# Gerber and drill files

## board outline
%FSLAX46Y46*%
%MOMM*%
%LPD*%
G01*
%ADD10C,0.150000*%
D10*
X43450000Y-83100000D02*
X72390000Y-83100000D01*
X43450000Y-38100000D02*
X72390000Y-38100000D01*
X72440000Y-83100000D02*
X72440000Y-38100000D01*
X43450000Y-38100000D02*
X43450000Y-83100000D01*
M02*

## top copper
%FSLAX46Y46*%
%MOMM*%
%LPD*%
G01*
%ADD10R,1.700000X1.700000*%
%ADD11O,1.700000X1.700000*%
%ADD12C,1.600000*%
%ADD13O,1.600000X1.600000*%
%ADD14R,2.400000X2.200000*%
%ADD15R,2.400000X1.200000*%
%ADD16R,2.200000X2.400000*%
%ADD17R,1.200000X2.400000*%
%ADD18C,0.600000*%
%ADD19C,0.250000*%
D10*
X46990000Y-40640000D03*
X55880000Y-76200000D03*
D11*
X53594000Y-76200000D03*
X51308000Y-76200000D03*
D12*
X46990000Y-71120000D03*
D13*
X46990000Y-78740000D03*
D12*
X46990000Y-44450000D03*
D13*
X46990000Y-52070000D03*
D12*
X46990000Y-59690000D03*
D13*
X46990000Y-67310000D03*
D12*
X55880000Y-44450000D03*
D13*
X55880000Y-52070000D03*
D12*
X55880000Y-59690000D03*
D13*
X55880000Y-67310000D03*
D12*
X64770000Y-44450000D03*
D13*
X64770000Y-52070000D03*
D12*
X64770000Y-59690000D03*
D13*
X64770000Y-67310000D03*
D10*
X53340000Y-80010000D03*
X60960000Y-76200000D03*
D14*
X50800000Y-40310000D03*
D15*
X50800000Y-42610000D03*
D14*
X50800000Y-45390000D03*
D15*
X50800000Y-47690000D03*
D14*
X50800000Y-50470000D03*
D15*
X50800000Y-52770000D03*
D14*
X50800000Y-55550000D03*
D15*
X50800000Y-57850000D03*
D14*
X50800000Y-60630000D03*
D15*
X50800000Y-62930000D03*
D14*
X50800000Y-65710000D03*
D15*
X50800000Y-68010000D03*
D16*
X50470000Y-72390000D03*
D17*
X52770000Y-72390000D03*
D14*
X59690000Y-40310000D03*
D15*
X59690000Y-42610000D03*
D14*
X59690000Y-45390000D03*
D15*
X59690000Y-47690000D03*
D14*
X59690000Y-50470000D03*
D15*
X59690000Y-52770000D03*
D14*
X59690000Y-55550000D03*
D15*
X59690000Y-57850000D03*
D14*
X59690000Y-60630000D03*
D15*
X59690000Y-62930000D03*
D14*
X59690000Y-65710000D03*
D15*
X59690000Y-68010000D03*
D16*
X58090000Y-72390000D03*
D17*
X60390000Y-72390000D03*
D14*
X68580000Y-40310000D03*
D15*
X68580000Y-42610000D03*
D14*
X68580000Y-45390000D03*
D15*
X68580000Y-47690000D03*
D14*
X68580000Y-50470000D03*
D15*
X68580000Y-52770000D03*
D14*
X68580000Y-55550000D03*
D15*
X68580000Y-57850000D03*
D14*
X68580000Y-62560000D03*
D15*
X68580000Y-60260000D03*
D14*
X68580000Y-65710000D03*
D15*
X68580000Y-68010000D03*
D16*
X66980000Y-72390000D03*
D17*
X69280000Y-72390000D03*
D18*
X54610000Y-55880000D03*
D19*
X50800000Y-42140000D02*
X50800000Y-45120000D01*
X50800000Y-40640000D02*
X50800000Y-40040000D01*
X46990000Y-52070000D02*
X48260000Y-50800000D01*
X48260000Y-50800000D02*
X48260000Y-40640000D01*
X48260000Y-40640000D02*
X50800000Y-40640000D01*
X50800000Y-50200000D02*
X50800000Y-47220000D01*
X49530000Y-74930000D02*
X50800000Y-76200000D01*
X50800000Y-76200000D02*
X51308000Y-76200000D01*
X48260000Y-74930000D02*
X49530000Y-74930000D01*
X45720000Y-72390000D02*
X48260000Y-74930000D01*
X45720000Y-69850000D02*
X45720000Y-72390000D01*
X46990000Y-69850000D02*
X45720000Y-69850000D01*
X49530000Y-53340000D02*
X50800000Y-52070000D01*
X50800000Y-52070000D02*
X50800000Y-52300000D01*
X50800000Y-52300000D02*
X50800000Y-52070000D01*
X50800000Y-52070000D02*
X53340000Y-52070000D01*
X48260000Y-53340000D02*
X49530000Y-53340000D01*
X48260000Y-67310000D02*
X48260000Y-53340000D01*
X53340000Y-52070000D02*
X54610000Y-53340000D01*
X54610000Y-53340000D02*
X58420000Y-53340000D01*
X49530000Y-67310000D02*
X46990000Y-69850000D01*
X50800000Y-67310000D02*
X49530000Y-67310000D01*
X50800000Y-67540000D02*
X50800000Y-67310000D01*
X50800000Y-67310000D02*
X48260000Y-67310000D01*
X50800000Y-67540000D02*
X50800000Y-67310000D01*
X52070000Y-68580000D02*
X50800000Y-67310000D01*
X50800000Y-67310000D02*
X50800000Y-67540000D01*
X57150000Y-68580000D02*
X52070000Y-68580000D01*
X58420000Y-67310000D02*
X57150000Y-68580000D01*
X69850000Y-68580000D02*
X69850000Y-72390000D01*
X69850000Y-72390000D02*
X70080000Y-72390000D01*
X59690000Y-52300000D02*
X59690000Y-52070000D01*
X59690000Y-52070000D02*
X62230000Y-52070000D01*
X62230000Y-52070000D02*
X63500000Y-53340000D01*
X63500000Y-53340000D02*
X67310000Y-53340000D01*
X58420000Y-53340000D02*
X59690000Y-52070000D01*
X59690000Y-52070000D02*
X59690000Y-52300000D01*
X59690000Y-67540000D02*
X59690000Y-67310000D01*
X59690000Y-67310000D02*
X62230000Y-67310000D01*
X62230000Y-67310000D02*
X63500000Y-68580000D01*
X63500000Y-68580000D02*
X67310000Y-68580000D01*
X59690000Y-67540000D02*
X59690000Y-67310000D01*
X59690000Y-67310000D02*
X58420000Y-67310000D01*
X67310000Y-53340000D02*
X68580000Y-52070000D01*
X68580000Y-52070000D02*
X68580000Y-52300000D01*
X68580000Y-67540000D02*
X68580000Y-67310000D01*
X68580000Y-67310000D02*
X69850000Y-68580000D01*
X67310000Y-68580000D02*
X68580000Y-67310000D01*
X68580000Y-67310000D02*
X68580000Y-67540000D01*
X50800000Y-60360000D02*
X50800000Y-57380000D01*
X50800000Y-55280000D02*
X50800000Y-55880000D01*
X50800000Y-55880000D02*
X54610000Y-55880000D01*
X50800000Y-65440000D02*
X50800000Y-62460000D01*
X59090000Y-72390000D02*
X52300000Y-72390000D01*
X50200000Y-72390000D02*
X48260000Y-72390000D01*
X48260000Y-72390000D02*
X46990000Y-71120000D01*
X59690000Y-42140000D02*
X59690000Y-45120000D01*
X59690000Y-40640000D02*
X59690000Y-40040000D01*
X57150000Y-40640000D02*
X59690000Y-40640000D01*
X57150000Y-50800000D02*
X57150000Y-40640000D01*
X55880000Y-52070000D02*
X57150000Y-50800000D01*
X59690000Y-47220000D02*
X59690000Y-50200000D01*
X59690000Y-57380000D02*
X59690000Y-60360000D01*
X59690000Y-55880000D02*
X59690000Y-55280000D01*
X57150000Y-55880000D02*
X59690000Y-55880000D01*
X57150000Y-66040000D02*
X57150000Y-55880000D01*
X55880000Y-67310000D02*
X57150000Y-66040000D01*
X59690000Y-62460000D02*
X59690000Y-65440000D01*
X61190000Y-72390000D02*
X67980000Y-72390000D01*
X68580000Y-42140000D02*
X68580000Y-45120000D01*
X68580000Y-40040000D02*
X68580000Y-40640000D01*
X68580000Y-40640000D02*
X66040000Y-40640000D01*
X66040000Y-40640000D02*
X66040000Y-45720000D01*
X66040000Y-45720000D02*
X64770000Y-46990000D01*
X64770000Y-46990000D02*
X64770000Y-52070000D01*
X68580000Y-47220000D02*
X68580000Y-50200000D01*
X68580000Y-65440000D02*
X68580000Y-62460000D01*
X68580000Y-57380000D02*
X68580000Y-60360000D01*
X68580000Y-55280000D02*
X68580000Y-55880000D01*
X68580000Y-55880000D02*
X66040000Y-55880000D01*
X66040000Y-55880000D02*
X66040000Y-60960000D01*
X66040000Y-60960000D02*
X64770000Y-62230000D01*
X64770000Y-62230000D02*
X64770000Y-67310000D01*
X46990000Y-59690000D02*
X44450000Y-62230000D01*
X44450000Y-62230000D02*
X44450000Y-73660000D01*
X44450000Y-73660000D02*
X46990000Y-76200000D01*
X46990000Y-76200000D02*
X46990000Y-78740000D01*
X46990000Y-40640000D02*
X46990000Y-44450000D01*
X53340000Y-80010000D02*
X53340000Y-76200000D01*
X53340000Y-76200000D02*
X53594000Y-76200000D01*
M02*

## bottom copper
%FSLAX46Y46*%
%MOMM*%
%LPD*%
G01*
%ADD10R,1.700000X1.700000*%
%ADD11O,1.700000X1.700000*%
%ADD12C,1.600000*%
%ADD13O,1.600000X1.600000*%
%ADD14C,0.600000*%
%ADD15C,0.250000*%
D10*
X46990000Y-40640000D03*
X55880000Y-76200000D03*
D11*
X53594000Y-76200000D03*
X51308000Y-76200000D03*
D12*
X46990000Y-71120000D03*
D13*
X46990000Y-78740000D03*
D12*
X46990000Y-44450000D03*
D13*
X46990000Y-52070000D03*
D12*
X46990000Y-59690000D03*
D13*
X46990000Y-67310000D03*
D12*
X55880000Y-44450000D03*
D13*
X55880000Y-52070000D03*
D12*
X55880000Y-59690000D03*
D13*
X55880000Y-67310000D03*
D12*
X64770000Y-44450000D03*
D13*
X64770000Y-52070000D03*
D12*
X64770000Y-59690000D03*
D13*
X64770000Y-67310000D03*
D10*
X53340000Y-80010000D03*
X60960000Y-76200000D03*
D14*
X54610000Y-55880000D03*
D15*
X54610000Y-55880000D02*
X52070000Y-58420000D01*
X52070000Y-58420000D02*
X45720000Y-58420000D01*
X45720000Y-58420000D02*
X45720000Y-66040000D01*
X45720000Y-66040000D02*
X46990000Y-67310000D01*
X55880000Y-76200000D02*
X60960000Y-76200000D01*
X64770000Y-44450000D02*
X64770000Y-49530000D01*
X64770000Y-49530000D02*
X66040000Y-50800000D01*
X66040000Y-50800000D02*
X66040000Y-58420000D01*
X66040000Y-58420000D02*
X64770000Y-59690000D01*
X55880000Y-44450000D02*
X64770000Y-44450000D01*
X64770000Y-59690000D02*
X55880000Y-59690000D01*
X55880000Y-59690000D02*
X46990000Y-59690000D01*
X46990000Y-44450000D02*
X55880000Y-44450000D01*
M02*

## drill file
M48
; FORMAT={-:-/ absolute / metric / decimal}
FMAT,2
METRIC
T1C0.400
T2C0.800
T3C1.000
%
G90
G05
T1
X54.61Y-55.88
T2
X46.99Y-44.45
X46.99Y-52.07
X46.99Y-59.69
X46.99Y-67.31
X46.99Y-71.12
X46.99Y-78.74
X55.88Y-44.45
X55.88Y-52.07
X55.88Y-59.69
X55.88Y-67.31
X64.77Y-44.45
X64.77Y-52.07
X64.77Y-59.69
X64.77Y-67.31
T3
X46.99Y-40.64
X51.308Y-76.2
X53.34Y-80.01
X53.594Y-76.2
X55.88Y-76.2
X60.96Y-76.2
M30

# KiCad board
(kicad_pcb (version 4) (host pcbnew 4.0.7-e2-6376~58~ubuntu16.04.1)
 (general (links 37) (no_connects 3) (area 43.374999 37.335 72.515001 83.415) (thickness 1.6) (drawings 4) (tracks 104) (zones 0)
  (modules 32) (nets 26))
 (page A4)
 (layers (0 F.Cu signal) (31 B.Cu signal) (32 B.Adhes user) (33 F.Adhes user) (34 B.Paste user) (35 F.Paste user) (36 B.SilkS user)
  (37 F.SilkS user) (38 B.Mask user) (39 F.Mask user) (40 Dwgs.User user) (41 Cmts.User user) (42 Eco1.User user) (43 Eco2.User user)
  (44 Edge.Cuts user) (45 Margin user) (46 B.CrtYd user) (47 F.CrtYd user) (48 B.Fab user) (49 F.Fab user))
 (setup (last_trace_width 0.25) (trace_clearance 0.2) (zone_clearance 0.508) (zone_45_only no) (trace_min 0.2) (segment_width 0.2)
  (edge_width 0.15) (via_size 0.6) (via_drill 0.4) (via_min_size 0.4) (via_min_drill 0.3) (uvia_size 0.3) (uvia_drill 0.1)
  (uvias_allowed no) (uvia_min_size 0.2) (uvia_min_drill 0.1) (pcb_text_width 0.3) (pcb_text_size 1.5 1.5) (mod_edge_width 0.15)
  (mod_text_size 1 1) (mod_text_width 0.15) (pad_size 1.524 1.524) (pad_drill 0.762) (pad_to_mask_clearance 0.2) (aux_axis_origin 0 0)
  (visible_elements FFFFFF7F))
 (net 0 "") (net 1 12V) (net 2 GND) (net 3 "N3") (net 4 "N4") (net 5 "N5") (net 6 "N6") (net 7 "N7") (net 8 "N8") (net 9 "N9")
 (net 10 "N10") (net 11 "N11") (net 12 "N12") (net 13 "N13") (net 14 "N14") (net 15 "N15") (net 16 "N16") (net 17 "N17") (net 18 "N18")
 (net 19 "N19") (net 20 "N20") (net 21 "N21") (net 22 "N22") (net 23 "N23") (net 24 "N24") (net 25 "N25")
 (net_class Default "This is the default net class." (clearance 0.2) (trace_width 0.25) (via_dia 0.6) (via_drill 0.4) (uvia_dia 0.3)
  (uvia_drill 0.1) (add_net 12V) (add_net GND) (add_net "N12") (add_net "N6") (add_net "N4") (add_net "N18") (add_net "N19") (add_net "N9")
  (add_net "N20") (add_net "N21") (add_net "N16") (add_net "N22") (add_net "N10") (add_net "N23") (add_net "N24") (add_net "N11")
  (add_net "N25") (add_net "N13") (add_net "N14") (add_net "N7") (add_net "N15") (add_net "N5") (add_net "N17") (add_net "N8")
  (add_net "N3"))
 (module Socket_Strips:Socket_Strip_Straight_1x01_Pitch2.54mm (layer F.Cu) (at 46.99 40.64)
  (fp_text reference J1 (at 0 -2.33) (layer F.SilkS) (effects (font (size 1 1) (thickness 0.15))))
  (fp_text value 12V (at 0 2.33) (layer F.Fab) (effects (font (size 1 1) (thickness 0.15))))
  (pad 1 thru_hole rect (at 0 0) (size 1.7 1.7) (drill 1) (layers *.Cu *.Mask) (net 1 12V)))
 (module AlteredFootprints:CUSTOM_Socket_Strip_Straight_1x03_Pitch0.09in (layer F.Cu) (at 55.88 76.2 270)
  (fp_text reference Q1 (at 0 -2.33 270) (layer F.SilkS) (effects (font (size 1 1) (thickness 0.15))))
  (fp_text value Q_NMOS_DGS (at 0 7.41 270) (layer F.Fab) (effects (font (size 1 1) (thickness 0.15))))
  (pad 1 thru_hole rect (at 0 0 270) (size 1.7 1.7) (drill 1) (layers *.Cu *.Mask) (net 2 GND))
  (pad 2 thru_hole oval (at 0 2.286 270) (size 1.7 1.7) (drill 1) (layers *.Cu *.Mask) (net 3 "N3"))
  (pad 3 thru_hole oval (at 0 4.572 270) (size 1.7 1.7) (drill 1) (layers *.Cu *.Mask) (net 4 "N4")))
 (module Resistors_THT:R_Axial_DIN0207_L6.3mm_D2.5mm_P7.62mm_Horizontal (layer F.Cu) (at 46.99 71.12 270)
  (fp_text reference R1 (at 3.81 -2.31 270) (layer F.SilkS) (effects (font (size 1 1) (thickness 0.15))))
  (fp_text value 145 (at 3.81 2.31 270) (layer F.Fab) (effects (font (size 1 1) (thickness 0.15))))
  (pad 1 thru_hole circle (at 0 0 270) (size 1.6 1.6) (drill 0.8) (layers *.Cu *.Mask) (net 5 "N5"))
  (pad 2 thru_hole oval (at 7.62 0 270) (size 1.6 1.6) (drill 0.8) (layers *.Cu *.Mask) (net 1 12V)))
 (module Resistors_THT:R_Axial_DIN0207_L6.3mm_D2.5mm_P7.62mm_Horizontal (layer F.Cu) (at 46.99 44.45 270)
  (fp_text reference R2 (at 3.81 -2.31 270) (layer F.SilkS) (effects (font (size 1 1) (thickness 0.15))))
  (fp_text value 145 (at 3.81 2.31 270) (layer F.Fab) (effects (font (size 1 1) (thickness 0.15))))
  (pad 1 thru_hole circle (at 0 0 270) (size 1.6 1.6) (drill 0.8) (layers *.Cu *.Mask) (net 1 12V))
  (pad 2 thru_hole oval (at 7.62 0 270) (size 1.6 1.6) (drill 0.8) (layers *.Cu *.Mask) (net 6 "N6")))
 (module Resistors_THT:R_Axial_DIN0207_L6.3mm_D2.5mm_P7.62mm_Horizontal (layer F.Cu) (at 46.99 59.69 270)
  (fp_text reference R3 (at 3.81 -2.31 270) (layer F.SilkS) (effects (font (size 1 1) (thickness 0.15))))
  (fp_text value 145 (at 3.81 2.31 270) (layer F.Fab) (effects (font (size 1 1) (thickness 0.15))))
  (pad 1 thru_hole circle (at 0 0 270) (size 1.6 1.6) (drill 0.8) (layers *.Cu *.Mask) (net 1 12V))
  (pad 2 thru_hole oval (at 7.62 0 270) (size 1.6 1.6) (drill 0.8) (layers *.Cu *.Mask) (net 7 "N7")))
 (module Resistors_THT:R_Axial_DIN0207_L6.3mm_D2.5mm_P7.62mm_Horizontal (layer F.Cu) (at 55.88 44.45 270)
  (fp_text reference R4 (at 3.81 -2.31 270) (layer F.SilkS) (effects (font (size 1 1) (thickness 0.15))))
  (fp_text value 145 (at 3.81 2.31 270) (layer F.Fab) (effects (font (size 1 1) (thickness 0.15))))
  (pad 1 thru_hole circle (at 0 0 270) (size 1.6 1.6) (drill 0.8) (layers *.Cu *.Mask) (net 1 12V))
  (pad 2 thru_hole oval (at 7.62 0 270) (size 1.6 1.6) (drill 0.8) (layers *.Cu *.Mask) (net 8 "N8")))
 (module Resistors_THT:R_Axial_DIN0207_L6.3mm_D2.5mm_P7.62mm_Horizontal (layer F.Cu) (at 55.88 59.69 270)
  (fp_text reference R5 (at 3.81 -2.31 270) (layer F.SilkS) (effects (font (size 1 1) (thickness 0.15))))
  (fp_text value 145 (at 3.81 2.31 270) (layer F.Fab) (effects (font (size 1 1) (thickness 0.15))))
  (pad 1 thru_hole circle (at 0 0 270) (size 1.6 1.6) (drill 0.8) (layers *.Cu *.Mask) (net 1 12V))
  (pad 2 thru_hole oval (at 7.62 0 270) (size 1.6 1.6) (drill 0.8) (layers *.Cu *.Mask) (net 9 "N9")))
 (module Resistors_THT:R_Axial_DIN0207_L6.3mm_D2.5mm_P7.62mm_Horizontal (layer F.Cu) (at 64.77 44.45 270)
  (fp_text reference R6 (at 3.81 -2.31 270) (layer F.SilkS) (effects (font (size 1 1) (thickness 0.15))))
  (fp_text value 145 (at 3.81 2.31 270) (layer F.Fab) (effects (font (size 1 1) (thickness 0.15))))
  (pad 1 thru_hole circle (at 0 0 270) (size 1.6 1.6) (drill 0.8) (layers *.Cu *.Mask) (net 1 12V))
  (pad 2 thru_hole oval (at 7.62 0 270) (size 1.6 1.6) (drill 0.8) (layers *.Cu *.Mask) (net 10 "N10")))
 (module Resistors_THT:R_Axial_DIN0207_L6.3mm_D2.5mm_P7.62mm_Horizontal (layer F.Cu) (at 64.77 59.69 270)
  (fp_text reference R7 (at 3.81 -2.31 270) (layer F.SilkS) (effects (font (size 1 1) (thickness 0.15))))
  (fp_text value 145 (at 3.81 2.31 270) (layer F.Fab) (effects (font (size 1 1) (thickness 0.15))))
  (pad 1 thru_hole circle (at 0 0 270) (size 1.6 1.6) (drill 0.8) (layers *.Cu *.Mask) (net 1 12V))
  (pad 2 thru_hole oval (at 7.62 0 270) (size 1.6 1.6) (drill 0.8) (layers *.Cu *.Mask) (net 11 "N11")))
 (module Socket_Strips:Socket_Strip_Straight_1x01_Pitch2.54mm (layer F.Cu) (at 53.34 80.01)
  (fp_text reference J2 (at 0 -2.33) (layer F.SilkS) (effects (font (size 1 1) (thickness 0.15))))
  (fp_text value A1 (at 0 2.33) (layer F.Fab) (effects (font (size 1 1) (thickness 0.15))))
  (pad 1 thru_hole rect (at 0 0) (size 1.7 1.7) (drill 1) (layers *.Cu *.Mask) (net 3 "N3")))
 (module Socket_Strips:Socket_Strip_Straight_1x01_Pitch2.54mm (layer F.Cu) (at 60.96 76.2)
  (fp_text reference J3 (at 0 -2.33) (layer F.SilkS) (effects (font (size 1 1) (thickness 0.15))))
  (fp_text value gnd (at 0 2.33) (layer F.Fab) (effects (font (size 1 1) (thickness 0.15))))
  (pad 1 thru_hole rect (at 0 0) (size 1.7 1.7) (drill 1) (layers *.Cu *.Mask) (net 2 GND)))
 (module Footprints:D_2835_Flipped (layer F.Cu) (at 50.8 41.91 90)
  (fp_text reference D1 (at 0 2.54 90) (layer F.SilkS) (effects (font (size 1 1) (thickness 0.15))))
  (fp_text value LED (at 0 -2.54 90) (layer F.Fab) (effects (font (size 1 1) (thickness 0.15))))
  (pad 2 smd rect (at 1.6 0 90) (size 2.2 2.4) (layers F.Cu F.Paste F.Mask) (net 6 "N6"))
  (pad 1 smd rect (at -0.7 0 90) (size 1.2 2.4) (layers F.Cu F.Paste F.Mask) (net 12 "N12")))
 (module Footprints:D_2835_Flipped (layer F.Cu) (at 50.8 46.99 90)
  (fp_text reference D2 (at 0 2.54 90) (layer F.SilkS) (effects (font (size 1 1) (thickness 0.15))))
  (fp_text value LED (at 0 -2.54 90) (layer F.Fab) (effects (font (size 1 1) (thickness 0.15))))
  (pad 2 smd rect (at 1.6 0 90) (size 2.2 2.4) (layers F.Cu F.Paste F.Mask) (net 12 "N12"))
  (pad 1 smd rect (at -0.7 0 90) (size 1.2 2.4) (layers F.Cu F.Paste F.Mask) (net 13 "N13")))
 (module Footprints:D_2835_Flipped (layer F.Cu) (at 50.8 52.07 90)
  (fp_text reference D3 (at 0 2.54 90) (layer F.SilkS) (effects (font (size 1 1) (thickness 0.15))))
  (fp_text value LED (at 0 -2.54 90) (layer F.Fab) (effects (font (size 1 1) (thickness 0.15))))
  (pad 2 smd rect (at 1.6 0 90) (size 2.2 2.4) (layers F.Cu F.Paste F.Mask) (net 13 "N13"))
  (pad 1 smd rect (at -0.7 0 90) (size 1.2 2.4) (layers F.Cu F.Paste F.Mask) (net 4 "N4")))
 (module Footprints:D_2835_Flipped (layer F.Cu) (at 50.8 57.15 90)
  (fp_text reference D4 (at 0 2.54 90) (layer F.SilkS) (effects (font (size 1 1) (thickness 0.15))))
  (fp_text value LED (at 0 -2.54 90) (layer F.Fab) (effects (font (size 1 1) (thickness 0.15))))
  (pad 2 smd rect (at 1.6 0 90) (size 2.2 2.4) (layers F.Cu F.Paste F.Mask) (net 7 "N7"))
  (pad 1 smd rect (at -0.7 0 90) (size 1.2 2.4) (layers F.Cu F.Paste F.Mask) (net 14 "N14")))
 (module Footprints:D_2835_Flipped (layer F.Cu) (at 50.8 62.23 90)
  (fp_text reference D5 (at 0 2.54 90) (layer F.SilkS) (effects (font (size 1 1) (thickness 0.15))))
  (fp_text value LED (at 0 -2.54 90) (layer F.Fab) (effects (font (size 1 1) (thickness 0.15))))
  (pad 2 smd rect (at 1.6 0 90) (size 2.2 2.4) (layers F.Cu F.Paste F.Mask) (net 14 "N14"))
  (pad 1 smd rect (at -0.7 0 90) (size 1.2 2.4) (layers F.Cu F.Paste F.Mask) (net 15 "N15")))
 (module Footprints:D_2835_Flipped (layer F.Cu) (at 50.8 67.31 90)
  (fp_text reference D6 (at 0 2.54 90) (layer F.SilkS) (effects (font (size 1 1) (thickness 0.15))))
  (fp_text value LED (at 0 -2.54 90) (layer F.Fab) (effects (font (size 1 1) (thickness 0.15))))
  (pad 2 smd rect (at 1.6 0 90) (size 2.2 2.4) (layers F.Cu F.Paste F.Mask) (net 15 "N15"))
  (pad 1 smd rect (at -0.7 0 90) (size 1.2 2.4) (layers F.Cu F.Paste F.Mask) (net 4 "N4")))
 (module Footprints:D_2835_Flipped (layer F.Cu) (at 52.07 72.39 180)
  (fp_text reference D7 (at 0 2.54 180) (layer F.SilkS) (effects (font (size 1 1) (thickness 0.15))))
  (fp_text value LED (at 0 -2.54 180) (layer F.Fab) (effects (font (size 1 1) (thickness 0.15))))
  (pad 2 smd rect (at 1.6 0 180) (size 2.2 2.4) (layers F.Cu F.Paste F.Mask) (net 5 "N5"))
  (pad 1 smd rect (at -0.7 0 180) (size 1.2 2.4) (layers F.Cu F.Paste F.Mask) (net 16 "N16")))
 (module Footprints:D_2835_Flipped (layer F.Cu) (at 59.69 41.91 90)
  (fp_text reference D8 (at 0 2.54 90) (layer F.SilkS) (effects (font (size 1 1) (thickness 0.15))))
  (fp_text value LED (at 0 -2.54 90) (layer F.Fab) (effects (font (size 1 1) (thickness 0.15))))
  (pad 2 smd rect (at 1.6 0 90) (size 2.2 2.4) (layers F.Cu F.Paste F.Mask) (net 8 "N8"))
  (pad 1 smd rect (at -0.7 0 90) (size 1.2 2.4) (layers F.Cu F.Paste F.Mask) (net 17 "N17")))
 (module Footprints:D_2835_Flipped (layer F.Cu) (at 59.69 46.99 90)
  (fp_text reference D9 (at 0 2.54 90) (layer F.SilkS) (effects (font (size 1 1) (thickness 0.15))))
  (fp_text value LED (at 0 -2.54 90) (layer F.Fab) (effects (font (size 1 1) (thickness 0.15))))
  (pad 2 smd rect (at 1.6 0 90) (size 2.2 2.4) (layers F.Cu F.Paste F.Mask) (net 17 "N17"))
  (pad 1 smd rect (at -0.7 0 90) (size 1.2 2.4) (layers F.Cu F.Paste F.Mask) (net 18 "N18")))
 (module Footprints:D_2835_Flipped (layer F.Cu) (at 59.69 52.07 90)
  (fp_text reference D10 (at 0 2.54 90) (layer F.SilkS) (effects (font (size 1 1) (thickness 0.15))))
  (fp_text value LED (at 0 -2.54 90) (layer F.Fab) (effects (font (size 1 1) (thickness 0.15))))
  (pad 2 smd rect (at 1.6 0 90) (size 2.2 2.4) (layers F.Cu F.Paste F.Mask) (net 18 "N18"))
  (pad 1 smd rect (at -0.7 0 90) (size 1.2 2.4) (layers F.Cu F.Paste F.Mask) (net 4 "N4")))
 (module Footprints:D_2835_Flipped (layer F.Cu) (at 59.69 57.15 90)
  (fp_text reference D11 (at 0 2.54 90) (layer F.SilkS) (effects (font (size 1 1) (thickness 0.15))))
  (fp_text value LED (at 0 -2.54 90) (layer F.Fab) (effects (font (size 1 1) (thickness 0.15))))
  (pad 2 smd rect (at 1.6 0 90) (size 2.2 2.4) (layers F.Cu F.Paste F.Mask) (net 9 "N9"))
  (pad 1 smd rect (at -0.7 0 90) (size 1.2 2.4) (layers F.Cu F.Paste F.Mask) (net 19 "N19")))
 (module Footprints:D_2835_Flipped (layer F.Cu) (at 59.69 62.23 90)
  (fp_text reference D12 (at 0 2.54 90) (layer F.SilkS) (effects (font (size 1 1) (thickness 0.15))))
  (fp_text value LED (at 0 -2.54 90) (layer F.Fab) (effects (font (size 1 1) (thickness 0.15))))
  (pad 2 smd rect (at 1.6 0 90) (size 2.2 2.4) (layers F.Cu F.Paste F.Mask) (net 19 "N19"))
  (pad 1 smd rect (at -0.7 0 90) (size 1.2 2.4) (layers F.Cu F.Paste F.Mask) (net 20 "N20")))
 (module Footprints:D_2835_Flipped (layer F.Cu) (at 59.69 67.31 90)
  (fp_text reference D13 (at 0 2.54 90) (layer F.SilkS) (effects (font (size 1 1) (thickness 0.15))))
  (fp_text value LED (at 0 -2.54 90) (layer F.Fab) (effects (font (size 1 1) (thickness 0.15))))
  (pad 2 smd rect (at 1.6 0 90) (size 2.2 2.4) (layers F.Cu F.Paste F.Mask) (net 20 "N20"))
  (pad 1 smd rect (at -0.7 0 90) (size 1.2 2.4) (layers F.Cu F.Paste F.Mask) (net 4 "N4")))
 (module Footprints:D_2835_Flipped (layer F.Cu) (at 59.69 72.39 180)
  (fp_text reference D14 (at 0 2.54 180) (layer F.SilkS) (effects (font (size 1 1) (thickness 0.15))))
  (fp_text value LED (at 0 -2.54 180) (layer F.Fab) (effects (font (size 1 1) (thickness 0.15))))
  (pad 2 smd rect (at 1.6 0 180) (size 2.2 2.4) (layers F.Cu F.Paste F.Mask) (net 16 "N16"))
  (pad 1 smd rect (at -0.7 0 180) (size 1.2 2.4) (layers F.Cu F.Paste F.Mask) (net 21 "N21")))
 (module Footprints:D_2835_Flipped (layer F.Cu) (at 68.58 41.91 90)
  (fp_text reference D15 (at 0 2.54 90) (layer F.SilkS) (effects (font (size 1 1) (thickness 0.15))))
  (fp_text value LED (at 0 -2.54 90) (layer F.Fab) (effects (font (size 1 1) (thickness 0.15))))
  (pad 2 smd rect (at 1.6 0 90) (size 2.2 2.4) (layers F.Cu F.Paste F.Mask) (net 10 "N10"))
  (pad 1 smd rect (at -0.7 0 90) (size 1.2 2.4) (layers F.Cu F.Paste F.Mask) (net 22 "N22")))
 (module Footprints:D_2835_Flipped (layer F.Cu) (at 68.58 46.99 90)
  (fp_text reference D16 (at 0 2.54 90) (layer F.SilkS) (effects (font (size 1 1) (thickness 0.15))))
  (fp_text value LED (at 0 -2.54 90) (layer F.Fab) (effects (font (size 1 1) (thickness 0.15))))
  (pad 2 smd rect (at 1.6 0 90) (size 2.2 2.4) (layers F.Cu F.Paste F.Mask) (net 22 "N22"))
  (pad 1 smd rect (at -0.7 0 90) (size 1.2 2.4) (layers F.Cu F.Paste F.Mask) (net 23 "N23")))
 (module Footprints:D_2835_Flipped (layer F.Cu) (at 68.58 52.07 90)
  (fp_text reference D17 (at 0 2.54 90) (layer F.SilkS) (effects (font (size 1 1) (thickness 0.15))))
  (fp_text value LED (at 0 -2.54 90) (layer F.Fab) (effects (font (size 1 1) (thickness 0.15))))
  (pad 2 smd rect (at 1.6 0 90) (size 2.2 2.4) (layers F.Cu F.Paste F.Mask) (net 23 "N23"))
  (pad 1 smd rect (at -0.7 0 90) (size 1.2 2.4) (layers F.Cu F.Paste F.Mask) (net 4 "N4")))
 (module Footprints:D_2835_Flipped (layer F.Cu) (at 68.58 57.15 90)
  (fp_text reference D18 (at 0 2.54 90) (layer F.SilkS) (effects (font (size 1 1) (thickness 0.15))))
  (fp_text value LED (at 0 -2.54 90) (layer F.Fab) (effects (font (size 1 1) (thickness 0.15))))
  (pad 2 smd rect (at 1.6 0 90) (size 2.2 2.4) (layers F.Cu F.Paste F.Mask) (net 11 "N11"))
  (pad 1 smd rect (at -0.7 0 90) (size 1.2 2.4) (layers F.Cu F.Paste F.Mask) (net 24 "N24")))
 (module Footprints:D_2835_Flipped (layer F.Cu) (at 68.58 60.96 270)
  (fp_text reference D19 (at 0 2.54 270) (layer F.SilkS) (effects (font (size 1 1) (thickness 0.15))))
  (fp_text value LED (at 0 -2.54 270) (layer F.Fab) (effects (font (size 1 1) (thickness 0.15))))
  (pad 2 smd rect (at 1.6 0 270) (size 2.2 2.4) (layers F.Cu F.Paste F.Mask) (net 24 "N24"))
  (pad 1 smd rect (at -0.7 0 270) (size 1.2 2.4) (layers F.Cu F.Paste F.Mask) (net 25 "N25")))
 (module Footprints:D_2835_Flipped (layer F.Cu) (at 68.58 67.31 90)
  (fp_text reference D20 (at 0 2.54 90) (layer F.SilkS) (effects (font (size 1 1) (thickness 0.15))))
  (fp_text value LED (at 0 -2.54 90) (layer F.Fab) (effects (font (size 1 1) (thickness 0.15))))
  (pad 2 smd rect (at 1.6 0 90) (size 2.2 2.4) (layers F.Cu F.Paste F.Mask) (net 25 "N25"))
  (pad 1 smd rect (at -0.7 0 90) (size 1.2 2.4) (layers F.Cu F.Paste F.Mask) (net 4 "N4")))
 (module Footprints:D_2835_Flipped (layer F.Cu) (at 68.58 72.39 180)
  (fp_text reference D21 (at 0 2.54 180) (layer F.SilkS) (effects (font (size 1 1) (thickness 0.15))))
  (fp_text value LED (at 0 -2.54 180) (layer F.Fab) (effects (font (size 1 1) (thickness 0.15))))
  (pad 2 smd rect (at 1.6 0 180) (size 2.2 2.4) (layers F.Cu F.Paste F.Mask) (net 21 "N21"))
  (pad 1 smd rect (at -0.7 0 180) (size 1.2 2.4) (layers F.Cu F.Paste F.Mask) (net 4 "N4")))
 (gr_line (start 43.45 83.1) (end 72.39 83.1) (angle 90) (layer Edge.Cuts) (width 0.15))
 (gr_line (start 43.45 38.1) (end 72.39 38.1) (angle 90) (layer Edge.Cuts) (width 0.15))
 (gr_line (start 72.44 83.1) (end 72.44 38.1) (angle 90) (layer Edge.Cuts) (width 0.15))
 (gr_line (start 43.45 38.1) (end 43.45 83.1) (angle 90) (layer Edge.Cuts) (width 0.15))
 (segment (start 50.8 42.14) (end 50.8 45.12) (width 0.25) (layer F.Cu) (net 12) (status 80000))
 (segment (start 50.8 40.64) (end 50.8 40.04) (width 0.25) (layer F.Cu) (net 6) (status 80000))
 (segment (start 46.99 52.07) (end 48.26 50.8) (width 0.25) (layer F.Cu) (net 6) (status 80000))
 (segment (start 48.26 50.8) (end 48.26 40.64) (width 0.25) (layer F.Cu) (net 6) (status 80000))
 (segment (start 48.26 40.64) (end 50.8 40.64) (width 0.25) (layer F.Cu) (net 6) (status 80000))
 (segment (start 50.8 50.2) (end 50.8 47.22) (width 0.25) (layer F.Cu) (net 13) (status 80000))
 (segment (start 49.53 74.93) (end 50.8 76.2) (width 0.25) (layer F.Cu) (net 4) (status 80000))
 (segment (start 50.8 76.2) (end 51.308 76.2) (width 0.25) (layer F.Cu) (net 4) (status 80000))
 (segment (start 48.26 74.93) (end 49.53 74.93) (width 0.25) (layer F.Cu) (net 4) (status 80000))
 (segment (start 45.72 72.39) (end 48.26 74.93) (width 0.25) (layer F.Cu) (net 4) (status 80000))
 (segment (start 45.72 69.85) (end 45.72 72.39) (width 0.25) (layer F.Cu) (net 4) (status 80000))
 (segment (start 46.99 69.85) (end 45.72 69.85) (width 0.25) (layer F.Cu) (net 4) (status 80000))
 (segment (start 49.53 53.34) (end 50.8 52.07) (width 0.25) (layer F.Cu) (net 4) (status 80000))
 (segment (start 50.8 52.07) (end 50.8 52.3) (width 0.25) (layer F.Cu) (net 4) (status 80000))
 (segment (start 50.8 52.3) (end 50.8 52.07) (width 0.25) (layer F.Cu) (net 4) (status 80000))
 (segment (start 50.8 52.07) (end 53.34 52.07) (width 0.25) (layer F.Cu) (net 4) (status 80000))
 (segment (start 48.26 53.34) (end 49.53 53.34) (width 0.25) (layer F.Cu) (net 4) (status 80000))
 (segment (start 48.26 67.31) (end 48.26 53.34) (width 0.25) (layer F.Cu) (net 4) (status 80000))
 (segment (start 53.34 52.07) (end 54.61 53.34) (width 0.25) (layer F.Cu) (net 4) (status 80000))
 (segment (start 54.61 53.34) (end 58.42 53.34) (width 0.25) (layer F.Cu) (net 4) (status 80000))
 (segment (start 49.53 67.31) (end 46.99 69.85) (width 0.25) (layer F.Cu) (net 4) (status 80000))
 (segment (start 50.8 67.31) (end 49.53 67.31) (width 0.25) (layer F.Cu) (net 4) (status 80000))
 (segment (start 50.8 67.54) (end 50.8 67.31) (width 0.25) (layer F.Cu) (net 4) (status 80000))
 (segment (start 50.8 67.31) (end 48.26 67.31) (width 0.25) (layer F.Cu) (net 4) (status 80000))
 (segment (start 50.8 67.54) (end 50.8 67.31) (width 0.25) (layer F.Cu) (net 4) (status 80000))
 (segment (start 52.07 68.58) (end 50.8 67.31) (width 0.25) (layer F.Cu) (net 4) (status 80000))
 (segment (start 50.8 67.31) (end 50.8 67.54) (width 0.25) (layer F.Cu) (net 4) (status 80000))
 (segment (start 57.15 68.58) (end 52.07 68.58) (width 0.25) (layer F.Cu) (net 4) (status 80000))
 (segment (start 58.42 67.31) (end 57.15 68.58) (width 0.25) (layer F.Cu) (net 4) (status 80000))
 (segment (start 69.85 68.58) (end 69.85 72.39) (width 0.25) (layer F.Cu) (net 4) (status 80000))
 (segment (start 69.85 72.39) (end 70.08 72.39) (width 0.25) (layer F.Cu) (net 4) (status 80000))
 (segment (start 59.69 52.3) (end 59.69 52.07) (width 0.25) (layer F.Cu) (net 4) (status 80000))
 (segment (start 59.69 52.07) (end 62.23 52.07) (width 0.25) (layer F.Cu) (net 4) (status 80000))
 (segment (start 62.23 52.07) (end 63.5 53.34) (width 0.25) (layer F.Cu) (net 4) (status 80000))
 (segment (start 63.5 53.34) (end 67.31 53.34) (width 0.25) (layer F.Cu) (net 4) (status 80000))
 (segment (start 58.42 53.34) (end 59.69 52.07) (width 0.25) (layer F.Cu) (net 4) (status 80000))
 (segment (start 59.69 52.07) (end 59.69 52.3) (width 0.25) (layer F.Cu) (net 4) (status 80000))
 (segment (start 59.69 67.54) (end 59.69 67.31) (width 0.25) (layer F.Cu) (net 4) (status 80000))
 (segment (start 59.69 67.31) (end 62.23 67.31) (width 0.25) (layer F.Cu) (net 4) (status 80000))
 (segment (start 62.23 67.31) (end 63.5 68.58) (width 0.25) (layer F.Cu) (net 4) (status 80000))
 (segment (start 63.5 68.58) (end 67.31 68.58) (width 0.25) (layer F.Cu) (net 4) (status 80000))
 (segment (start 59.69 67.54) (end 59.69 67.31) (width 0.25) (layer F.Cu) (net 4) (status 80000))
 (segment (start 59.69 67.31) (end 58.42 67.31) (width 0.25) (layer F.Cu) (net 4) (status 80000))
 (segment (start 67.31 53.34) (end 68.58 52.07) (width 0.25) (layer F.Cu) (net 4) (status 80000))
 (segment (start 68.58 52.07) (end 68.58 52.3) (width 0.25) (layer F.Cu) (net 4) (status 80000))
 (segment (start 68.58 67.54) (end 68.58 67.31) (width 0.25) (layer F.Cu) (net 4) (status 80000))
 (segment (start 68.58 67.31) (end 69.85 68.58) (width 0.25) (layer F.Cu) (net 4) (status 80000))
 (segment (start 67.31 68.58) (end 68.58 67.31) (width 0.25) (layer F.Cu) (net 4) (status 80000))
 (segment (start 68.58 67.31) (end 68.58 67.54) (width 0.25) (layer F.Cu) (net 4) (status 80000))
 (segment (start 50.8 60.36) (end 50.8 57.38) (width 0.25) (layer F.Cu) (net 14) (status 80000))
 (segment (start 50.8 55.28) (end 50.8 55.88) (width 0.25) (layer F.Cu) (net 7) (status 80000))
 (segment (start 50.8 55.88) (end 54.61 55.88) (width 0.25) (layer F.Cu) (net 7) (status 80000))
 (via (at 54.61 55.88) (size 0.6) (layers F.Cu B.Cu) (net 7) (status 80000))
 (segment (start 54.61 55.88) (end 52.07 58.42) (width 0.25) (layer B.Cu) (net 7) (status 80000))
 (segment (start 52.07 58.42) (end 45.72 58.42) (width 0.25) (layer B.Cu) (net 7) (status 80000))
 (segment (start 45.72 58.42) (end 45.72 66.04) (width 0.25) (layer B.Cu) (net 7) (status 80000))
 (segment (start 45.72 66.04) (end 46.99 67.31) (width 0.25) (layer B.Cu) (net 7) (status 80000))
 (segment (start 50.8 65.44) (end 50.8 62.46) (width 0.25) (layer F.Cu) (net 15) (status 80000))
 (segment (start 59.09 72.39) (end 52.3 72.39) (width 0.25) (layer F.Cu) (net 16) (status 80000))
 (segment (start 50.2 72.39) (end 48.26 72.39) (width 0.25) (layer F.Cu) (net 5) (status 80000))
 (segment (start 48.26 72.39) (end 46.99 71.12) (width 0.25) (layer F.Cu) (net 5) (status 80000))
 (segment (start 59.69 42.14) (end 59.69 45.12) (width 0.25) (layer F.Cu) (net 17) (status 80000))
 (segment (start 59.69 40.64) (end 59.69 40.04) (width 0.25) (layer F.Cu) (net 8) (status 80000))
 (segment (start 57.15 40.64) (end 59.69 40.64) (width 0.25) (layer F.Cu) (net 8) (status 80000))
 (segment (start 57.15 50.8) (end 57.15 40.64) (width 0.25) (layer F.Cu) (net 8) (status 80000))
 (segment (start 55.88 52.07) (end 57.15 50.8) (width 0.25) (layer F.Cu) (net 8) (status 80000))
 (segment (start 59.69 47.22) (end 59.69 50.2) (width 0.25) (layer F.Cu) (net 18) (status 80000))
 (segment (start 59.69 57.38) (end 59.69 60.36) (width 0.25) (layer F.Cu) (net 19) (status 80000))
 (segment (start 59.69 55.88) (end 59.69 55.28) (width 0.25) (layer F.Cu) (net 9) (status 80000))
 (segment (start 57.15 55.88) (end 59.69 55.88) (width 0.25) (layer F.Cu) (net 9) (status 80000))
 (segment (start 57.15 66.04) (end 57.15 55.88) (width 0.25) (layer F.Cu) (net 9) (status 80000))
 (segment (start 55.88 67.31) (end 57.15 66.04) (width 0.25) (layer F.Cu) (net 9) (status 80000))
 (segment (start 59.69 62.46) (end 59.69 65.44) (width 0.25) (layer F.Cu) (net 20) (status 80000))
 (segment (start 61.19 72.39) (end 67.98 72.39) (width 0.25) (layer F.Cu) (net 21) (status 80000))
 (segment (start 68.58 42.14) (end 68.58 45.12) (width 0.25) (layer F.Cu) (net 22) (status 80000))
 (segment (start 68.58 40.04) (end 68.58 40.64) (width 0.25) (layer F.Cu) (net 10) (status 80000))
 (segment (start 68.58 40.64) (end 66.04 40.64) (width 0.25) (layer F.Cu) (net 10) (status 80000))
 (segment (start 66.04 40.64) (end 66.04 45.72) (width 0.25) (layer F.Cu) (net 10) (status 80000))
 (segment (start 66.04 45.72) (end 64.77 46.99) (width 0.25) (layer F.Cu) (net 10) (status 80000))
 (segment (start 64.77 46.99) (end 64.77 52.07) (width 0.25) (layer F.Cu) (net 10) (status 80000))
 (segment (start 68.58 47.22) (end 68.58 50.2) (width 0.25) (layer F.Cu) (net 23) (status 80000))
 (segment (start 68.58 65.44) (end 68.58 62.46) (width 0.25) (layer F.Cu) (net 24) (status 80000))
 (segment (start 68.58 57.38) (end 68.58 60.36) (width 0.25) (layer F.Cu) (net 24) (status 80000))
 (segment (start 68.58 55.28) (end 68.58 55.88) (width 0.25) (layer F.Cu) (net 11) (status 80000))
 (segment (start 68.58 55.88) (end 66.04 55.88) (width 0.25) (layer F.Cu) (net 11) (status 80000))
 (segment (start 66.04 55.88) (end 66.04 60.96) (width 0.25) (layer F.Cu) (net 11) (status 80000))
 (segment (start 66.04 60.96) (end 64.77 62.23) (width 0.25) (layer F.Cu) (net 11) (status 80000))
 (segment (start 64.77 62.23) (end 64.77 67.31) (width 0.25) (layer F.Cu) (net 11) (status 80000))
 (segment (start 55.88 76.2) (end 60.96 76.2) (width 0.25) (layer B.Cu) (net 2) (status 80000))
 (segment (start 46.99 59.69) (end 44.45 62.23) (width 0.25) (layer F.Cu) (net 1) (status 80000))
 (segment (start 44.45 62.23) (end 44.45 73.66) (width 0.25) (layer F.Cu) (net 1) (status 80000))
 (segment (start 44.45 73.66) (end 46.99 76.2) (width 0.25) (layer F.Cu) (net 1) (status 80000))
 (segment (start 46.99 76.2) (end 46.99 78.74) (width 0.25) (layer F.Cu) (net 1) (status 80000))
 (segment (start 64.77 44.45) (end 64.77 49.53) (width 0.25) (layer B.Cu) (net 1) (status 80000))
 (segment (start 64.77 49.53) (end 66.04 50.8) (width 0.25) (layer B.Cu) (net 1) (status 80000))
 (segment (start 66.04 50.8) (end 66.04 58.42) (width 0.25) (layer B.Cu) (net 1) (status 80000))
 (segment (start 66.04 58.42) (end 64.77 59.69) (width 0.25) (layer B.Cu) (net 1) (status 80000))
 (segment (start 55.88 44.45) (end 64.77 44.45) (width 0.25) (layer B.Cu) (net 1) (status 80000))
 (segment (start 64.77 59.69) (end 55.88 59.69) (width 0.25) (layer B.Cu) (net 1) (status 80000))
 (segment (start 55.88 59.69) (end 46.99 59.69) (width 0.25) (layer B.Cu) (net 1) (status 80000))
 (segment (start 46.99 44.45) (end 55.88 44.45) (width 0.25) (layer B.Cu) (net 1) (status 80000))
 (segment (start 46.99 40.64) (end 46.99 44.45) (width 0.25) (layer F.Cu) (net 1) (status 80000))
 (segment (start 53.34 80.01) (end 53.34 76.2) (width 0.25) (layer F.Cu) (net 3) (status 80000))
 (segment (start 53.34 76.2) (end 53.594 76.2) (width 0.25) (layer F.Cu) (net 3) (status 80000)))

